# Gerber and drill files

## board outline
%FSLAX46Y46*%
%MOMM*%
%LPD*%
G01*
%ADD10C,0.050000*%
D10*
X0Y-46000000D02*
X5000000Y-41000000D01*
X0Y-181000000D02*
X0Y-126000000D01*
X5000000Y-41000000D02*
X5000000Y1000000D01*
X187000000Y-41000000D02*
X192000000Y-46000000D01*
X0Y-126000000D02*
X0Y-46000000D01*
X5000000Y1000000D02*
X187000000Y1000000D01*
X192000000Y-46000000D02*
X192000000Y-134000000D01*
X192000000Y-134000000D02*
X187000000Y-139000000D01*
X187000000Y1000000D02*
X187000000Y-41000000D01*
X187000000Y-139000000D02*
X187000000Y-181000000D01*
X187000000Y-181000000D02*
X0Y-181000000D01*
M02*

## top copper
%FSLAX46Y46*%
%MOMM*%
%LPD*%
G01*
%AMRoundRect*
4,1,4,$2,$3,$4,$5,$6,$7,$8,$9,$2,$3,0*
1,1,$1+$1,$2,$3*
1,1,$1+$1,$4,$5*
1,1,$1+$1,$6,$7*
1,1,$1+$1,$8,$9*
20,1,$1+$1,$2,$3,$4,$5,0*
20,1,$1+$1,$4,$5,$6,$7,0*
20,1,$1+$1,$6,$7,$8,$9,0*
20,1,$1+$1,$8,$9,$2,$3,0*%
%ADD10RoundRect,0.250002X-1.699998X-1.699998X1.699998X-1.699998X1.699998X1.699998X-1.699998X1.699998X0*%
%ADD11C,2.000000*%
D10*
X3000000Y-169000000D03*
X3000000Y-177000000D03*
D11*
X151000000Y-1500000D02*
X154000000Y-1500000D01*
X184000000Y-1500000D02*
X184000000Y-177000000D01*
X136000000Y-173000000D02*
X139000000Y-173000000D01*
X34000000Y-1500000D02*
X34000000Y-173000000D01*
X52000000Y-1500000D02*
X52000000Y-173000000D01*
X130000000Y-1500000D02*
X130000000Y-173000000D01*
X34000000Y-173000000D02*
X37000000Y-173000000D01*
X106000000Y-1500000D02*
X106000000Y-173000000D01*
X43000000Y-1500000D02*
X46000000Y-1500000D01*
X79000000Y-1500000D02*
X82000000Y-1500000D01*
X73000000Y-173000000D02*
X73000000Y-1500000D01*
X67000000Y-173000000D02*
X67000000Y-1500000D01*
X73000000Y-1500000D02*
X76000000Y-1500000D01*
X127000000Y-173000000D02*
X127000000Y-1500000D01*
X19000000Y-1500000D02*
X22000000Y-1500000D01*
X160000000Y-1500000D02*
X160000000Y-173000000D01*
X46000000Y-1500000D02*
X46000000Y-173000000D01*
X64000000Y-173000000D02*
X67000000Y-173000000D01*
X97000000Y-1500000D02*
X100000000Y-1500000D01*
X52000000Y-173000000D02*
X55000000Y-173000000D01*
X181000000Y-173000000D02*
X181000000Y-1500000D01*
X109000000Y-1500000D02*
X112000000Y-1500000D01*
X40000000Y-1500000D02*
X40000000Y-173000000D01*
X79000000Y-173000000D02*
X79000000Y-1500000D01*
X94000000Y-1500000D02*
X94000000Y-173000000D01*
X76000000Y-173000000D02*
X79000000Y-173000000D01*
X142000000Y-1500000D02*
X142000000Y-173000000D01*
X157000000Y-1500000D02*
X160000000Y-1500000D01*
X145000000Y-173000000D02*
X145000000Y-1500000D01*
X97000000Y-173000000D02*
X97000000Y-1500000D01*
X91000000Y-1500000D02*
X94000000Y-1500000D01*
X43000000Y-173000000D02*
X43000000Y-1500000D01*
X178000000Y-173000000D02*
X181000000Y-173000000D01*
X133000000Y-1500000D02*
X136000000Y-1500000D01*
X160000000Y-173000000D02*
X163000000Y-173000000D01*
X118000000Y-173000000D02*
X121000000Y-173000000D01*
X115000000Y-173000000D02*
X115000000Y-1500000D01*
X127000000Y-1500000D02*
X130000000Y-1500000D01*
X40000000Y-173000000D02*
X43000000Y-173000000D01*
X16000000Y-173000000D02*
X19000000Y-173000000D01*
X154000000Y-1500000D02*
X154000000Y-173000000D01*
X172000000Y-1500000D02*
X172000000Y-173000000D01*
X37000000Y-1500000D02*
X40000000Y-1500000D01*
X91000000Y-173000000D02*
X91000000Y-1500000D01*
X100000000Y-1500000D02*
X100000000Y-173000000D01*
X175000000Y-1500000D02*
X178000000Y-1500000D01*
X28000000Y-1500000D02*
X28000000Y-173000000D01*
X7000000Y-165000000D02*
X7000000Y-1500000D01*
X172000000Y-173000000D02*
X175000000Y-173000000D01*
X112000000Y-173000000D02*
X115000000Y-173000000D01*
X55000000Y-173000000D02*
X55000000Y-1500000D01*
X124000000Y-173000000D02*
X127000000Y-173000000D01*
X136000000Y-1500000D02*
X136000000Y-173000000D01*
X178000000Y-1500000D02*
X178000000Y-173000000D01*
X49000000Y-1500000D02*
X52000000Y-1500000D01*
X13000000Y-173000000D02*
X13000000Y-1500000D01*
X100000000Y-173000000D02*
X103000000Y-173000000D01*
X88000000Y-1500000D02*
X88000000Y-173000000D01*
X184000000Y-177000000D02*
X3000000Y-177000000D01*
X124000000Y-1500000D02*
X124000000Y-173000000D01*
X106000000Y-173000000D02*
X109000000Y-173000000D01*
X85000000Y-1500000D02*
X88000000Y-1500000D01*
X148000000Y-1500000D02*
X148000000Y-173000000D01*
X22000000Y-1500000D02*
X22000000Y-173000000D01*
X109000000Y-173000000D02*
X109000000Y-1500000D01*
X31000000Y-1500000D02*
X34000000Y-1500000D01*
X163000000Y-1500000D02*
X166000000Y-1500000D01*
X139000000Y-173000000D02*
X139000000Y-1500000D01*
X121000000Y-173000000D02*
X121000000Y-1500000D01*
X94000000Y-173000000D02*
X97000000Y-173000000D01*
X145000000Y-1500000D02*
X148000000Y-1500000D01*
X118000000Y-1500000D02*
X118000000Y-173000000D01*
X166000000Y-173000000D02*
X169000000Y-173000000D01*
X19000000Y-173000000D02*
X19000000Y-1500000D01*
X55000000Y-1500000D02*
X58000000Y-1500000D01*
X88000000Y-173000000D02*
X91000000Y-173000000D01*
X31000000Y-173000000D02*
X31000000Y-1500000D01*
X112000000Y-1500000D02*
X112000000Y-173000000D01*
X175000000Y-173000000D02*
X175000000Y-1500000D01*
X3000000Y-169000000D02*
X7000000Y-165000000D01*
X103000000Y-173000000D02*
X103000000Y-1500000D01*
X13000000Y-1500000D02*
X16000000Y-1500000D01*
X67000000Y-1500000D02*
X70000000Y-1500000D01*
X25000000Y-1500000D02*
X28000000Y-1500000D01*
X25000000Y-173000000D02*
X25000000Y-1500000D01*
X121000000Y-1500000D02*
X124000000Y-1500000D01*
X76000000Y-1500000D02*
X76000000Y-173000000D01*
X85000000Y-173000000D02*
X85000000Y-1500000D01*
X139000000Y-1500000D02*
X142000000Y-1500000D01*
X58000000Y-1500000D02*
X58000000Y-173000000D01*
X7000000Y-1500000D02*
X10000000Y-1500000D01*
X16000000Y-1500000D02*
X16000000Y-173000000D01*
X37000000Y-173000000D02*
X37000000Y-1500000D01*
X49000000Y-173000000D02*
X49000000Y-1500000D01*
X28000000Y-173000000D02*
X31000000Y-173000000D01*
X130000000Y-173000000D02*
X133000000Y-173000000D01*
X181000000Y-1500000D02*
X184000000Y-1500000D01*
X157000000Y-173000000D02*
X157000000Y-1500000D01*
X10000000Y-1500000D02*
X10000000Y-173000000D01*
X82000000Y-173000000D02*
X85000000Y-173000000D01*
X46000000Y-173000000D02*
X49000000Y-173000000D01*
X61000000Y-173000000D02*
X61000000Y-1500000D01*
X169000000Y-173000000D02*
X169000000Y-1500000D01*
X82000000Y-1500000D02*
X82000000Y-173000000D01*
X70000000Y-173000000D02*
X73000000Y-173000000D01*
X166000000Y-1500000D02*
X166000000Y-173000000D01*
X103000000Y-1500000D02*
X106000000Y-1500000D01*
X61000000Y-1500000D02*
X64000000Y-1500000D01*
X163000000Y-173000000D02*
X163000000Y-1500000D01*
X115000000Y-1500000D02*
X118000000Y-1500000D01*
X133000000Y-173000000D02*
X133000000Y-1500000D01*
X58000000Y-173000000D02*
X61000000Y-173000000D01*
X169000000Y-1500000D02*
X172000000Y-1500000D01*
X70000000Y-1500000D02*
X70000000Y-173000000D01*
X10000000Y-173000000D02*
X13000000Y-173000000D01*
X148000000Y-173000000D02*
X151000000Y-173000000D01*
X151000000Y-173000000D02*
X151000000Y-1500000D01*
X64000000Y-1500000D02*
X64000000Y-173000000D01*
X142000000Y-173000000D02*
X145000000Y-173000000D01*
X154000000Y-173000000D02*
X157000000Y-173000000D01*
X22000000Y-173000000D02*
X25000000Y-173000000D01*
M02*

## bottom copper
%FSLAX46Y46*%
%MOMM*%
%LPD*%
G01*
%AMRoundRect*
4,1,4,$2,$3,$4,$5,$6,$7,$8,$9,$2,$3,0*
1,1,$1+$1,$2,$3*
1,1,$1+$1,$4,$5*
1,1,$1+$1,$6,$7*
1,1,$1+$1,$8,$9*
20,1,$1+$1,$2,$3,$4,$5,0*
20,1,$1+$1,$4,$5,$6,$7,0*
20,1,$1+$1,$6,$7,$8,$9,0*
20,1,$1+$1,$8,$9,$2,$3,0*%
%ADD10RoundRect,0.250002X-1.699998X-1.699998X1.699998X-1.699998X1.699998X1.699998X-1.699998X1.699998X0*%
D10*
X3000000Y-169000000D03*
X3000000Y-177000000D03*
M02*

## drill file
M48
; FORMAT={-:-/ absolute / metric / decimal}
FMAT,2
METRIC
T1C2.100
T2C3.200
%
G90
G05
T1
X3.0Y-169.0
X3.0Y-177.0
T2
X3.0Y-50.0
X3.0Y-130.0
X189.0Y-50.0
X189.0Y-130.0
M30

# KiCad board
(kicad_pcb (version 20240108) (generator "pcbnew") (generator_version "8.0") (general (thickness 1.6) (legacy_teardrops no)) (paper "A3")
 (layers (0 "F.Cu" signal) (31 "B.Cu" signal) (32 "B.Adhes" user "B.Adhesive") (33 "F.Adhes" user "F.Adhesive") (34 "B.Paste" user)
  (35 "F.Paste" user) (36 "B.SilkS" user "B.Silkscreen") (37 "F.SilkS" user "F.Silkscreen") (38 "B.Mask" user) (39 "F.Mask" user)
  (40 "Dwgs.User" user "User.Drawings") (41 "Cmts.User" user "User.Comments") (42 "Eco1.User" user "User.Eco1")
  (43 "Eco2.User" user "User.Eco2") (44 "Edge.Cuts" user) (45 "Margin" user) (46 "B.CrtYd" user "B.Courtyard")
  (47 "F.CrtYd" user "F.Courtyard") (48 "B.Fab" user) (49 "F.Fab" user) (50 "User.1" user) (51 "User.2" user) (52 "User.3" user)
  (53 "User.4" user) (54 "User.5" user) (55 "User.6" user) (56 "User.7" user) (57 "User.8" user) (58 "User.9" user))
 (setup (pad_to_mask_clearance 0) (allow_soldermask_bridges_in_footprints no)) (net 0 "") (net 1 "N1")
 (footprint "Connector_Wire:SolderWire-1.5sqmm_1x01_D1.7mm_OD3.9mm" (layer "F.Cu") (at 3 169)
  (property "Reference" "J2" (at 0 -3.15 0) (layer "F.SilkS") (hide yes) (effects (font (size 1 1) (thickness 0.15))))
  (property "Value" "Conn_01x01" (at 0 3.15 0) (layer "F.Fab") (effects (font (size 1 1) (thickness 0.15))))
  (pad "1" thru_hole roundrect (at 0 0) (size 3.9 3.9) (drill 2.1) (layers "*.Cu" "*.Mask") (remove_unused_layers no)
   (roundrect_rratio 0.064103) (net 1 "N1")))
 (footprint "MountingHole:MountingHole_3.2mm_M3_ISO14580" (layer "F.Cu") (at 189 50)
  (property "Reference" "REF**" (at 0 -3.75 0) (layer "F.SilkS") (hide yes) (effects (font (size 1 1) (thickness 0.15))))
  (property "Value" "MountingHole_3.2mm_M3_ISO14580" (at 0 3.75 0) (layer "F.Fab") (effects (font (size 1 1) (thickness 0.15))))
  (pad "" np_thru_hole circle (at 0 0) (size 3.2 3.2) (drill 3.2) (layers "*.Cu" "*.Mask")))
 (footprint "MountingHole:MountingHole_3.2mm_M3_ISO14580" (layer "F.Cu") (at 3 130)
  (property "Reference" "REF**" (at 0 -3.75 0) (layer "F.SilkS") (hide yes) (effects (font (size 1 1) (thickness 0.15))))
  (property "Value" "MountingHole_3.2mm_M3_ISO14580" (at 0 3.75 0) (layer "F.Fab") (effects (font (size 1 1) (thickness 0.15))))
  (pad "" np_thru_hole circle (at 0 0) (size 3.2 3.2) (drill 3.2) (layers "*.Cu" "*.Mask")))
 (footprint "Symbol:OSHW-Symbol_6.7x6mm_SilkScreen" (layer "F.Cu") (at 12 175)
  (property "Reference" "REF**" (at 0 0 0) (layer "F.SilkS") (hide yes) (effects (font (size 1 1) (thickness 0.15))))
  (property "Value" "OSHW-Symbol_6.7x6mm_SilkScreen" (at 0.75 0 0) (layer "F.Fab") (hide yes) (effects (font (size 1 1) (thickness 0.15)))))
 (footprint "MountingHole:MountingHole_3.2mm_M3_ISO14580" (layer "F.Cu") (at 189 130)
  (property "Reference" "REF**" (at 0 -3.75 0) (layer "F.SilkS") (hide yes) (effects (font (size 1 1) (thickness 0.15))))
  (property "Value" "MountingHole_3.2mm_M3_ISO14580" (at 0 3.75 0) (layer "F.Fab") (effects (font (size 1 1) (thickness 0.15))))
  (pad "" np_thru_hole circle (at 0 0) (size 3.2 3.2) (drill 3.2) (layers "*.Cu" "*.Mask")))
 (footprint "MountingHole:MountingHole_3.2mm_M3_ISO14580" (layer "F.Cu") (at 3 50)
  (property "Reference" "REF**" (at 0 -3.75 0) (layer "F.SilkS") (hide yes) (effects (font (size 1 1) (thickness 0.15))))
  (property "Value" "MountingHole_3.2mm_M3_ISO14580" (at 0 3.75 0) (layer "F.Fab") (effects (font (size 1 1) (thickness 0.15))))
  (pad "" np_thru_hole circle (at 0 0) (size 3.2 3.2) (drill 3.2) (layers "*.Cu" "*.Mask")))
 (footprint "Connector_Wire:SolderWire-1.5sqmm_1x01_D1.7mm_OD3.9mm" (layer "F.Cu") (at 3 177)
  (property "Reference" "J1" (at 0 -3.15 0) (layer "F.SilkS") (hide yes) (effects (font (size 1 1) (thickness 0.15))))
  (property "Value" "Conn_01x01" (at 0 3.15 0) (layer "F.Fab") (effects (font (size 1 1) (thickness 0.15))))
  (pad "1" thru_hole roundrect (at 0 0) (size 3.9 3.9) (drill 2.1) (layers "*.Cu" "*.Mask") (remove_unused_layers no)
   (roundrect_rratio 0.064103) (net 1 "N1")))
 (gr_line (start 0 46) (end 5 41) (stroke (width 0.05) (type default)) (layer "Edge.Cuts"))
 (gr_line (start 0 181) (end 0 126) (stroke (width 0.05) (type default)) (layer "Edge.Cuts"))
 (gr_line (start 5 41) (end 5 -1) (stroke (width 0.05) (type default)) (layer "Edge.Cuts"))
 (gr_line (start 187 41) (end 192 46) (stroke (width 0.05) (type default)) (layer "Edge.Cuts"))
 (gr_line (start 0 126) (end 0 46) (stroke (width 0.05) (type default)) (layer "Edge.Cuts"))
 (gr_line (start 5 -1) (end 187 -1) (stroke (width 0.05) (type default)) (layer "Edge.Cuts"))
 (gr_line (start 192 46) (end 192 134) (stroke (width 0.05) (type default)) (layer "Edge.Cuts"))
 (gr_line (start 192 134) (end 187 139) (stroke (width 0.05) (type default)) (layer "Edge.Cuts"))
 (gr_line (start 187 -1) (end 187 41) (stroke (width 0.05) (type default)) (layer "Edge.Cuts"))
 (gr_line (start 187 139) (end 187 181) (stroke (width 0.05) (type default)) (layer "Edge.Cuts"))
 (gr_line (start 187 181) (end 0 181) (stroke (width 0.05) (type default)) (layer "Edge.Cuts"))
 (segment (start 151 1.5) (end 154 1.5) (width 2) (layer "F.Cu") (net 1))
 (segment (start 184 1.5) (end 184 177) (width 2) (layer "F.Cu") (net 1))
 (segment (start 136 173) (end 139 173) (width 2) (layer "F.Cu") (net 1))
 (segment (start 34 1.5) (end 34 173) (width 2) (layer "F.Cu") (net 1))
 (segment (start 52 1.5) (end 52 173) (width 2) (layer "F.Cu") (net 1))
 (segment (start 130 1.5) (end 130 173) (width 2) (layer "F.Cu") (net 1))
 (segment (start 34 173) (end 37 173) (width 2) (layer "F.Cu") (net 1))
 (segment (start 106 1.5) (end 106 173) (width 2) (layer "F.Cu") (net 1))
 (segment (start 43 1.5) (end 46 1.5) (width 2) (layer "F.Cu") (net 1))
 (segment (start 79 1.5) (end 82 1.5) (width 2) (layer "F.Cu") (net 1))
 (segment (start 73 173) (end 73 1.5) (width 2) (layer "F.Cu") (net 1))
 (segment (start 67 173) (end 67 1.5) (width 2) (layer "F.Cu") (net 1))
 (segment (start 73 1.5) (end 76 1.5) (width 2) (layer "F.Cu") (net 1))
 (segment (start 127 173) (end 127 1.5) (width 2) (layer "F.Cu") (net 1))
 (segment (start 19 1.5) (end 22 1.5) (width 2) (layer "F.Cu") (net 1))
 (segment (start 160 1.5) (end 160 173) (width 2) (layer "F.Cu") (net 1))
 (segment (start 46 1.5) (end 46 173) (width 2) (layer "F.Cu") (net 1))
 (segment (start 64 173) (end 67 173) (width 2) (layer "F.Cu") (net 1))
 (segment (start 97 1.5) (end 100 1.5) (width 2) (layer "F.Cu") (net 1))
 (segment (start 52 173) (end 55 173) (width 2) (layer "F.Cu") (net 1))
 (segment (start 181 173) (end 181 1.5) (width 2) (layer "F.Cu") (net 1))
 (segment (start 109 1.5) (end 112 1.5) (width 2) (layer "F.Cu") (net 1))
 (segment (start 40 1.5) (end 40 173) (width 2) (layer "F.Cu") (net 1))
 (segment (start 79 173) (end 79 1.5) (width 2) (layer "F.Cu") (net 1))
 (segment (start 94 1.5) (end 94 173) (width 2) (layer "F.Cu") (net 1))
 (segment (start 76 173) (end 79 173) (width 2) (layer "F.Cu") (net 1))
 (segment (start 142 1.5) (end 142 173) (width 2) (layer "F.Cu") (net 1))
 (segment (start 157 1.5) (end 160 1.5) (width 2) (layer "F.Cu") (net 1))
 (segment (start 145 173) (end 145 1.5) (width 2) (layer "F.Cu") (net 1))
 (segment (start 97 173) (end 97 1.5) (width 2) (layer "F.Cu") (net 1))
 (segment (start 91 1.5) (end 94 1.5) (width 2) (layer "F.Cu") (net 1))
 (segment (start 43 173) (end 43 1.5) (width 2) (layer "F.Cu") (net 1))
 (segment (start 178 173) (end 181 173) (width 2) (layer "F.Cu") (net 1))
 (segment (start 133 1.5) (end 136 1.5) (width 2) (layer "F.Cu") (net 1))
 (segment (start 160 173) (end 163 173) (width 2) (layer "F.Cu") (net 1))
 (segment (start 118 173) (end 121 173) (width 2) (layer "F.Cu") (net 1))
 (segment (start 115 173) (end 115 1.5) (width 2) (layer "F.Cu") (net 1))
 (segment (start 127 1.5) (end 130 1.5) (width 2) (layer "F.Cu") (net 1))
 (segment (start 40 173) (end 43 173) (width 2) (layer "F.Cu") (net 1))
 (segment (start 16 173) (end 19 173) (width 2) (layer "F.Cu") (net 1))
 (segment (start 154 1.5) (end 154 173) (width 2) (layer "F.Cu") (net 1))
 (segment (start 172 1.5) (end 172 173) (width 2) (layer "F.Cu") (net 1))
 (segment (start 37 1.5) (end 40 1.5) (width 2) (layer "F.Cu") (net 1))
 (segment (start 91 173) (end 91 1.5) (width 2) (layer "F.Cu") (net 1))
 (segment (start 100 1.5) (end 100 173) (width 2) (layer "F.Cu") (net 1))
 (segment (start 175 1.5) (end 178 1.5) (width 2) (layer "F.Cu") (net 1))
 (segment (start 28 1.5) (end 28 173) (width 2) (layer "F.Cu") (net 1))
 (segment (start 7 165) (end 7 1.5) (width 2) (layer "F.Cu") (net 1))
 (segment (start 172 173) (end 175 173) (width 2) (layer "F.Cu") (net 1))
 (segment (start 112 173) (end 115 173) (width 2) (layer "F.Cu") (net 1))
 (segment (start 55 173) (end 55 1.5) (width 2) (layer "F.Cu") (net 1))
 (segment (start 124 173) (end 127 173) (width 2) (layer "F.Cu") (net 1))
 (segment (start 136 1.5) (end 136 173) (width 2) (layer "F.Cu") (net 1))
 (segment (start 178 1.5) (end 178 173) (width 2) (layer "F.Cu") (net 1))
 (segment (start 49 1.5) (end 52 1.5) (width 2) (layer "F.Cu") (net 1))
 (segment (start 13 173) (end 13 1.5) (width 2) (layer "F.Cu") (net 1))
 (segment (start 100 173) (end 103 173) (width 2) (layer "F.Cu") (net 1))
 (segment (start 88 1.5) (end 88 173) (width 2) (layer "F.Cu") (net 1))
 (segment (start 184 177) (end 3 177) (width 2) (layer "F.Cu") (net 1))
 (segment (start 124 1.5) (end 124 173) (width 2) (layer "F.Cu") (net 1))
 (segment (start 106 173) (end 109 173) (width 2) (layer "F.Cu") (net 1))
 (segment (start 85 1.5) (end 88 1.5) (width 2) (layer "F.Cu") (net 1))
 (segment (start 148 1.5) (end 148 173) (width 2) (layer "F.Cu") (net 1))
 (segment (start 22 1.5) (end 22 173) (width 2) (layer "F.Cu") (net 1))
 (segment (start 109 173) (end 109 1.5) (width 2) (layer "F.Cu") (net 1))
 (segment (start 31 1.5) (end 34 1.5) (width 2) (layer "F.Cu") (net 1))
 (segment (start 163 1.5) (end 166 1.5) (width 2) (layer "F.Cu") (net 1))
 (segment (start 139 173) (end 139 1.5) (width 2) (layer "F.Cu") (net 1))
 (segment (start 121 173) (end 121 1.5) (width 2) (layer "F.Cu") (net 1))
 (segment (start 94 173) (end 97 173) (width 2) (layer "F.Cu") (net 1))
 (segment (start 145 1.5) (end 148 1.5) (width 2) (layer "F.Cu") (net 1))
 (segment (start 118 1.5) (end 118 173) (width 2) (layer "F.Cu") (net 1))
 (segment (start 166 173) (end 169 173) (width 2) (layer "F.Cu") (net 1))
 (segment (start 19 173) (end 19 1.5) (width 2) (layer "F.Cu") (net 1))
 (segment (start 55 1.5) (end 58 1.5) (width 2) (layer "F.Cu") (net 1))
 (segment (start 88 173) (end 91 173) (width 2) (layer "F.Cu") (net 1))
 (segment (start 31 173) (end 31 1.5) (width 2) (layer "F.Cu") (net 1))
 (segment (start 112 1.5) (end 112 173) (width 2) (layer "F.Cu") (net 1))
 (segment (start 175 173) (end 175 1.5) (width 2) (layer "F.Cu") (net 1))
 (segment (start 3 169) (end 7 165) (width 2) (layer "F.Cu") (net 1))
 (segment (start 103 173) (end 103 1.5) (width 2) (layer "F.Cu") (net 1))
 (segment (start 13 1.5) (end 16 1.5) (width 2) (layer "F.Cu") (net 1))
 (segment (start 67 1.5) (end 70 1.5) (width 2) (layer "F.Cu") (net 1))
 (segment (start 25 1.5) (end 28 1.5) (width 2) (layer "F.Cu") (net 1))
 (segment (start 25 173) (end 25 1.5) (width 2) (layer "F.Cu") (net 1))
 (segment (start 121 1.5) (end 124 1.5) (width 2) (layer "F.Cu") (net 1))
 (segment (start 76 1.5) (end 76 173) (width 2) (layer "F.Cu") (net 1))
 (segment (start 85 173) (end 85 1.5) (width 2) (layer "F.Cu") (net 1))
 (segment (start 139 1.5) (end 142 1.5) (width 2) (layer "F.Cu") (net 1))
 (segment (start 58 1.5) (end 58 173) (width 2) (layer "F.Cu") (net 1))
 (segment (start 7 1.5) (end 10 1.5) (width 2) (layer "F.Cu") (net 1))
 (segment (start 16 1.5) (end 16 173) (width 2) (layer "F.Cu") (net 1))
 (segment (start 37 173) (end 37 1.5) (width 2) (layer "F.Cu") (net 1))
 (segment (start 49 173) (end 49 1.5) (width 2) (layer "F.Cu") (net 1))
 (segment (start 28 173) (end 31 173) (width 2) (layer "F.Cu") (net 1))
 (segment (start 130 173) (end 133 173) (width 2) (layer "F.Cu") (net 1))
 (segment (start 181 1.5) (end 184 1.5) (width 2) (layer "F.Cu") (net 1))
 (segment (start 157 173) (end 157 1.5) (width 2) (layer "F.Cu") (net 1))
 (segment (start 10 1.5) (end 10 173) (width 2) (layer "F.Cu") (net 1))
 (segment (start 82 173) (end 85 173) (width 2) (layer "F.Cu") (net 1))
 (segment (start 46 173) (end 49 173) (width 2) (layer "F.Cu") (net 1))
 (segment (start 61 173) (end 61 1.5) (width 2) (layer "F.Cu") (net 1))
 (segment (start 169 173) (end 169 1.5) (width 2) (layer "F.Cu") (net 1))
 (segment (start 82 1.5) (end 82 173) (width 2) (layer "F.Cu") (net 1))
 (segment (start 70 173) (end 73 173) (width 2) (layer "F.Cu") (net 1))
 (segment (start 166 1.5) (end 166 173) (width 2) (layer "F.Cu") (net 1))
 (segment (start 103 1.5) (end 106 1.5) (width 2) (layer "F.Cu") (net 1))
 (segment (start 61 1.5) (end 64 1.5) (width 2) (layer "F.Cu") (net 1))
 (segment (start 163 173) (end 163 1.5) (width 2) (layer "F.Cu") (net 1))
 (segment (start 115 1.5) (end 118 1.5) (width 2) (layer "F.Cu") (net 1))
 (segment (start 133 173) (end 133 1.5) (width 2) (layer "F.Cu") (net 1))
 (segment (start 58 173) (end 61 173) (width 2) (layer "F.Cu") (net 1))
 (segment (start 169 1.5) (end 172 1.5) (width 2) (layer "F.Cu") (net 1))
 (segment (start 70 1.5) (end 70 173) (width 2) (layer "F.Cu") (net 1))
 (segment (start 10 173) (end 13 173) (width 2) (layer "F.Cu") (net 1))
 (segment (start 148 173) (end 151 173) (width 2) (layer "F.Cu") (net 1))
 (segment (start 151 173) (end 151 1.5) (width 2) (layer "F.Cu") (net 1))
 (segment (start 64 1.5) (end 64 173) (width 2) (layer "F.Cu") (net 1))
 (segment (start 142 173) (end 145 173) (width 2) (layer "F.Cu") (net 1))
 (segment (start 154 173) (end 157 173) (width 2) (layer "F.Cu") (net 1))
 (segment (start 22 173) (end 25 173) (width 2) (layer "F.Cu") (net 1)))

